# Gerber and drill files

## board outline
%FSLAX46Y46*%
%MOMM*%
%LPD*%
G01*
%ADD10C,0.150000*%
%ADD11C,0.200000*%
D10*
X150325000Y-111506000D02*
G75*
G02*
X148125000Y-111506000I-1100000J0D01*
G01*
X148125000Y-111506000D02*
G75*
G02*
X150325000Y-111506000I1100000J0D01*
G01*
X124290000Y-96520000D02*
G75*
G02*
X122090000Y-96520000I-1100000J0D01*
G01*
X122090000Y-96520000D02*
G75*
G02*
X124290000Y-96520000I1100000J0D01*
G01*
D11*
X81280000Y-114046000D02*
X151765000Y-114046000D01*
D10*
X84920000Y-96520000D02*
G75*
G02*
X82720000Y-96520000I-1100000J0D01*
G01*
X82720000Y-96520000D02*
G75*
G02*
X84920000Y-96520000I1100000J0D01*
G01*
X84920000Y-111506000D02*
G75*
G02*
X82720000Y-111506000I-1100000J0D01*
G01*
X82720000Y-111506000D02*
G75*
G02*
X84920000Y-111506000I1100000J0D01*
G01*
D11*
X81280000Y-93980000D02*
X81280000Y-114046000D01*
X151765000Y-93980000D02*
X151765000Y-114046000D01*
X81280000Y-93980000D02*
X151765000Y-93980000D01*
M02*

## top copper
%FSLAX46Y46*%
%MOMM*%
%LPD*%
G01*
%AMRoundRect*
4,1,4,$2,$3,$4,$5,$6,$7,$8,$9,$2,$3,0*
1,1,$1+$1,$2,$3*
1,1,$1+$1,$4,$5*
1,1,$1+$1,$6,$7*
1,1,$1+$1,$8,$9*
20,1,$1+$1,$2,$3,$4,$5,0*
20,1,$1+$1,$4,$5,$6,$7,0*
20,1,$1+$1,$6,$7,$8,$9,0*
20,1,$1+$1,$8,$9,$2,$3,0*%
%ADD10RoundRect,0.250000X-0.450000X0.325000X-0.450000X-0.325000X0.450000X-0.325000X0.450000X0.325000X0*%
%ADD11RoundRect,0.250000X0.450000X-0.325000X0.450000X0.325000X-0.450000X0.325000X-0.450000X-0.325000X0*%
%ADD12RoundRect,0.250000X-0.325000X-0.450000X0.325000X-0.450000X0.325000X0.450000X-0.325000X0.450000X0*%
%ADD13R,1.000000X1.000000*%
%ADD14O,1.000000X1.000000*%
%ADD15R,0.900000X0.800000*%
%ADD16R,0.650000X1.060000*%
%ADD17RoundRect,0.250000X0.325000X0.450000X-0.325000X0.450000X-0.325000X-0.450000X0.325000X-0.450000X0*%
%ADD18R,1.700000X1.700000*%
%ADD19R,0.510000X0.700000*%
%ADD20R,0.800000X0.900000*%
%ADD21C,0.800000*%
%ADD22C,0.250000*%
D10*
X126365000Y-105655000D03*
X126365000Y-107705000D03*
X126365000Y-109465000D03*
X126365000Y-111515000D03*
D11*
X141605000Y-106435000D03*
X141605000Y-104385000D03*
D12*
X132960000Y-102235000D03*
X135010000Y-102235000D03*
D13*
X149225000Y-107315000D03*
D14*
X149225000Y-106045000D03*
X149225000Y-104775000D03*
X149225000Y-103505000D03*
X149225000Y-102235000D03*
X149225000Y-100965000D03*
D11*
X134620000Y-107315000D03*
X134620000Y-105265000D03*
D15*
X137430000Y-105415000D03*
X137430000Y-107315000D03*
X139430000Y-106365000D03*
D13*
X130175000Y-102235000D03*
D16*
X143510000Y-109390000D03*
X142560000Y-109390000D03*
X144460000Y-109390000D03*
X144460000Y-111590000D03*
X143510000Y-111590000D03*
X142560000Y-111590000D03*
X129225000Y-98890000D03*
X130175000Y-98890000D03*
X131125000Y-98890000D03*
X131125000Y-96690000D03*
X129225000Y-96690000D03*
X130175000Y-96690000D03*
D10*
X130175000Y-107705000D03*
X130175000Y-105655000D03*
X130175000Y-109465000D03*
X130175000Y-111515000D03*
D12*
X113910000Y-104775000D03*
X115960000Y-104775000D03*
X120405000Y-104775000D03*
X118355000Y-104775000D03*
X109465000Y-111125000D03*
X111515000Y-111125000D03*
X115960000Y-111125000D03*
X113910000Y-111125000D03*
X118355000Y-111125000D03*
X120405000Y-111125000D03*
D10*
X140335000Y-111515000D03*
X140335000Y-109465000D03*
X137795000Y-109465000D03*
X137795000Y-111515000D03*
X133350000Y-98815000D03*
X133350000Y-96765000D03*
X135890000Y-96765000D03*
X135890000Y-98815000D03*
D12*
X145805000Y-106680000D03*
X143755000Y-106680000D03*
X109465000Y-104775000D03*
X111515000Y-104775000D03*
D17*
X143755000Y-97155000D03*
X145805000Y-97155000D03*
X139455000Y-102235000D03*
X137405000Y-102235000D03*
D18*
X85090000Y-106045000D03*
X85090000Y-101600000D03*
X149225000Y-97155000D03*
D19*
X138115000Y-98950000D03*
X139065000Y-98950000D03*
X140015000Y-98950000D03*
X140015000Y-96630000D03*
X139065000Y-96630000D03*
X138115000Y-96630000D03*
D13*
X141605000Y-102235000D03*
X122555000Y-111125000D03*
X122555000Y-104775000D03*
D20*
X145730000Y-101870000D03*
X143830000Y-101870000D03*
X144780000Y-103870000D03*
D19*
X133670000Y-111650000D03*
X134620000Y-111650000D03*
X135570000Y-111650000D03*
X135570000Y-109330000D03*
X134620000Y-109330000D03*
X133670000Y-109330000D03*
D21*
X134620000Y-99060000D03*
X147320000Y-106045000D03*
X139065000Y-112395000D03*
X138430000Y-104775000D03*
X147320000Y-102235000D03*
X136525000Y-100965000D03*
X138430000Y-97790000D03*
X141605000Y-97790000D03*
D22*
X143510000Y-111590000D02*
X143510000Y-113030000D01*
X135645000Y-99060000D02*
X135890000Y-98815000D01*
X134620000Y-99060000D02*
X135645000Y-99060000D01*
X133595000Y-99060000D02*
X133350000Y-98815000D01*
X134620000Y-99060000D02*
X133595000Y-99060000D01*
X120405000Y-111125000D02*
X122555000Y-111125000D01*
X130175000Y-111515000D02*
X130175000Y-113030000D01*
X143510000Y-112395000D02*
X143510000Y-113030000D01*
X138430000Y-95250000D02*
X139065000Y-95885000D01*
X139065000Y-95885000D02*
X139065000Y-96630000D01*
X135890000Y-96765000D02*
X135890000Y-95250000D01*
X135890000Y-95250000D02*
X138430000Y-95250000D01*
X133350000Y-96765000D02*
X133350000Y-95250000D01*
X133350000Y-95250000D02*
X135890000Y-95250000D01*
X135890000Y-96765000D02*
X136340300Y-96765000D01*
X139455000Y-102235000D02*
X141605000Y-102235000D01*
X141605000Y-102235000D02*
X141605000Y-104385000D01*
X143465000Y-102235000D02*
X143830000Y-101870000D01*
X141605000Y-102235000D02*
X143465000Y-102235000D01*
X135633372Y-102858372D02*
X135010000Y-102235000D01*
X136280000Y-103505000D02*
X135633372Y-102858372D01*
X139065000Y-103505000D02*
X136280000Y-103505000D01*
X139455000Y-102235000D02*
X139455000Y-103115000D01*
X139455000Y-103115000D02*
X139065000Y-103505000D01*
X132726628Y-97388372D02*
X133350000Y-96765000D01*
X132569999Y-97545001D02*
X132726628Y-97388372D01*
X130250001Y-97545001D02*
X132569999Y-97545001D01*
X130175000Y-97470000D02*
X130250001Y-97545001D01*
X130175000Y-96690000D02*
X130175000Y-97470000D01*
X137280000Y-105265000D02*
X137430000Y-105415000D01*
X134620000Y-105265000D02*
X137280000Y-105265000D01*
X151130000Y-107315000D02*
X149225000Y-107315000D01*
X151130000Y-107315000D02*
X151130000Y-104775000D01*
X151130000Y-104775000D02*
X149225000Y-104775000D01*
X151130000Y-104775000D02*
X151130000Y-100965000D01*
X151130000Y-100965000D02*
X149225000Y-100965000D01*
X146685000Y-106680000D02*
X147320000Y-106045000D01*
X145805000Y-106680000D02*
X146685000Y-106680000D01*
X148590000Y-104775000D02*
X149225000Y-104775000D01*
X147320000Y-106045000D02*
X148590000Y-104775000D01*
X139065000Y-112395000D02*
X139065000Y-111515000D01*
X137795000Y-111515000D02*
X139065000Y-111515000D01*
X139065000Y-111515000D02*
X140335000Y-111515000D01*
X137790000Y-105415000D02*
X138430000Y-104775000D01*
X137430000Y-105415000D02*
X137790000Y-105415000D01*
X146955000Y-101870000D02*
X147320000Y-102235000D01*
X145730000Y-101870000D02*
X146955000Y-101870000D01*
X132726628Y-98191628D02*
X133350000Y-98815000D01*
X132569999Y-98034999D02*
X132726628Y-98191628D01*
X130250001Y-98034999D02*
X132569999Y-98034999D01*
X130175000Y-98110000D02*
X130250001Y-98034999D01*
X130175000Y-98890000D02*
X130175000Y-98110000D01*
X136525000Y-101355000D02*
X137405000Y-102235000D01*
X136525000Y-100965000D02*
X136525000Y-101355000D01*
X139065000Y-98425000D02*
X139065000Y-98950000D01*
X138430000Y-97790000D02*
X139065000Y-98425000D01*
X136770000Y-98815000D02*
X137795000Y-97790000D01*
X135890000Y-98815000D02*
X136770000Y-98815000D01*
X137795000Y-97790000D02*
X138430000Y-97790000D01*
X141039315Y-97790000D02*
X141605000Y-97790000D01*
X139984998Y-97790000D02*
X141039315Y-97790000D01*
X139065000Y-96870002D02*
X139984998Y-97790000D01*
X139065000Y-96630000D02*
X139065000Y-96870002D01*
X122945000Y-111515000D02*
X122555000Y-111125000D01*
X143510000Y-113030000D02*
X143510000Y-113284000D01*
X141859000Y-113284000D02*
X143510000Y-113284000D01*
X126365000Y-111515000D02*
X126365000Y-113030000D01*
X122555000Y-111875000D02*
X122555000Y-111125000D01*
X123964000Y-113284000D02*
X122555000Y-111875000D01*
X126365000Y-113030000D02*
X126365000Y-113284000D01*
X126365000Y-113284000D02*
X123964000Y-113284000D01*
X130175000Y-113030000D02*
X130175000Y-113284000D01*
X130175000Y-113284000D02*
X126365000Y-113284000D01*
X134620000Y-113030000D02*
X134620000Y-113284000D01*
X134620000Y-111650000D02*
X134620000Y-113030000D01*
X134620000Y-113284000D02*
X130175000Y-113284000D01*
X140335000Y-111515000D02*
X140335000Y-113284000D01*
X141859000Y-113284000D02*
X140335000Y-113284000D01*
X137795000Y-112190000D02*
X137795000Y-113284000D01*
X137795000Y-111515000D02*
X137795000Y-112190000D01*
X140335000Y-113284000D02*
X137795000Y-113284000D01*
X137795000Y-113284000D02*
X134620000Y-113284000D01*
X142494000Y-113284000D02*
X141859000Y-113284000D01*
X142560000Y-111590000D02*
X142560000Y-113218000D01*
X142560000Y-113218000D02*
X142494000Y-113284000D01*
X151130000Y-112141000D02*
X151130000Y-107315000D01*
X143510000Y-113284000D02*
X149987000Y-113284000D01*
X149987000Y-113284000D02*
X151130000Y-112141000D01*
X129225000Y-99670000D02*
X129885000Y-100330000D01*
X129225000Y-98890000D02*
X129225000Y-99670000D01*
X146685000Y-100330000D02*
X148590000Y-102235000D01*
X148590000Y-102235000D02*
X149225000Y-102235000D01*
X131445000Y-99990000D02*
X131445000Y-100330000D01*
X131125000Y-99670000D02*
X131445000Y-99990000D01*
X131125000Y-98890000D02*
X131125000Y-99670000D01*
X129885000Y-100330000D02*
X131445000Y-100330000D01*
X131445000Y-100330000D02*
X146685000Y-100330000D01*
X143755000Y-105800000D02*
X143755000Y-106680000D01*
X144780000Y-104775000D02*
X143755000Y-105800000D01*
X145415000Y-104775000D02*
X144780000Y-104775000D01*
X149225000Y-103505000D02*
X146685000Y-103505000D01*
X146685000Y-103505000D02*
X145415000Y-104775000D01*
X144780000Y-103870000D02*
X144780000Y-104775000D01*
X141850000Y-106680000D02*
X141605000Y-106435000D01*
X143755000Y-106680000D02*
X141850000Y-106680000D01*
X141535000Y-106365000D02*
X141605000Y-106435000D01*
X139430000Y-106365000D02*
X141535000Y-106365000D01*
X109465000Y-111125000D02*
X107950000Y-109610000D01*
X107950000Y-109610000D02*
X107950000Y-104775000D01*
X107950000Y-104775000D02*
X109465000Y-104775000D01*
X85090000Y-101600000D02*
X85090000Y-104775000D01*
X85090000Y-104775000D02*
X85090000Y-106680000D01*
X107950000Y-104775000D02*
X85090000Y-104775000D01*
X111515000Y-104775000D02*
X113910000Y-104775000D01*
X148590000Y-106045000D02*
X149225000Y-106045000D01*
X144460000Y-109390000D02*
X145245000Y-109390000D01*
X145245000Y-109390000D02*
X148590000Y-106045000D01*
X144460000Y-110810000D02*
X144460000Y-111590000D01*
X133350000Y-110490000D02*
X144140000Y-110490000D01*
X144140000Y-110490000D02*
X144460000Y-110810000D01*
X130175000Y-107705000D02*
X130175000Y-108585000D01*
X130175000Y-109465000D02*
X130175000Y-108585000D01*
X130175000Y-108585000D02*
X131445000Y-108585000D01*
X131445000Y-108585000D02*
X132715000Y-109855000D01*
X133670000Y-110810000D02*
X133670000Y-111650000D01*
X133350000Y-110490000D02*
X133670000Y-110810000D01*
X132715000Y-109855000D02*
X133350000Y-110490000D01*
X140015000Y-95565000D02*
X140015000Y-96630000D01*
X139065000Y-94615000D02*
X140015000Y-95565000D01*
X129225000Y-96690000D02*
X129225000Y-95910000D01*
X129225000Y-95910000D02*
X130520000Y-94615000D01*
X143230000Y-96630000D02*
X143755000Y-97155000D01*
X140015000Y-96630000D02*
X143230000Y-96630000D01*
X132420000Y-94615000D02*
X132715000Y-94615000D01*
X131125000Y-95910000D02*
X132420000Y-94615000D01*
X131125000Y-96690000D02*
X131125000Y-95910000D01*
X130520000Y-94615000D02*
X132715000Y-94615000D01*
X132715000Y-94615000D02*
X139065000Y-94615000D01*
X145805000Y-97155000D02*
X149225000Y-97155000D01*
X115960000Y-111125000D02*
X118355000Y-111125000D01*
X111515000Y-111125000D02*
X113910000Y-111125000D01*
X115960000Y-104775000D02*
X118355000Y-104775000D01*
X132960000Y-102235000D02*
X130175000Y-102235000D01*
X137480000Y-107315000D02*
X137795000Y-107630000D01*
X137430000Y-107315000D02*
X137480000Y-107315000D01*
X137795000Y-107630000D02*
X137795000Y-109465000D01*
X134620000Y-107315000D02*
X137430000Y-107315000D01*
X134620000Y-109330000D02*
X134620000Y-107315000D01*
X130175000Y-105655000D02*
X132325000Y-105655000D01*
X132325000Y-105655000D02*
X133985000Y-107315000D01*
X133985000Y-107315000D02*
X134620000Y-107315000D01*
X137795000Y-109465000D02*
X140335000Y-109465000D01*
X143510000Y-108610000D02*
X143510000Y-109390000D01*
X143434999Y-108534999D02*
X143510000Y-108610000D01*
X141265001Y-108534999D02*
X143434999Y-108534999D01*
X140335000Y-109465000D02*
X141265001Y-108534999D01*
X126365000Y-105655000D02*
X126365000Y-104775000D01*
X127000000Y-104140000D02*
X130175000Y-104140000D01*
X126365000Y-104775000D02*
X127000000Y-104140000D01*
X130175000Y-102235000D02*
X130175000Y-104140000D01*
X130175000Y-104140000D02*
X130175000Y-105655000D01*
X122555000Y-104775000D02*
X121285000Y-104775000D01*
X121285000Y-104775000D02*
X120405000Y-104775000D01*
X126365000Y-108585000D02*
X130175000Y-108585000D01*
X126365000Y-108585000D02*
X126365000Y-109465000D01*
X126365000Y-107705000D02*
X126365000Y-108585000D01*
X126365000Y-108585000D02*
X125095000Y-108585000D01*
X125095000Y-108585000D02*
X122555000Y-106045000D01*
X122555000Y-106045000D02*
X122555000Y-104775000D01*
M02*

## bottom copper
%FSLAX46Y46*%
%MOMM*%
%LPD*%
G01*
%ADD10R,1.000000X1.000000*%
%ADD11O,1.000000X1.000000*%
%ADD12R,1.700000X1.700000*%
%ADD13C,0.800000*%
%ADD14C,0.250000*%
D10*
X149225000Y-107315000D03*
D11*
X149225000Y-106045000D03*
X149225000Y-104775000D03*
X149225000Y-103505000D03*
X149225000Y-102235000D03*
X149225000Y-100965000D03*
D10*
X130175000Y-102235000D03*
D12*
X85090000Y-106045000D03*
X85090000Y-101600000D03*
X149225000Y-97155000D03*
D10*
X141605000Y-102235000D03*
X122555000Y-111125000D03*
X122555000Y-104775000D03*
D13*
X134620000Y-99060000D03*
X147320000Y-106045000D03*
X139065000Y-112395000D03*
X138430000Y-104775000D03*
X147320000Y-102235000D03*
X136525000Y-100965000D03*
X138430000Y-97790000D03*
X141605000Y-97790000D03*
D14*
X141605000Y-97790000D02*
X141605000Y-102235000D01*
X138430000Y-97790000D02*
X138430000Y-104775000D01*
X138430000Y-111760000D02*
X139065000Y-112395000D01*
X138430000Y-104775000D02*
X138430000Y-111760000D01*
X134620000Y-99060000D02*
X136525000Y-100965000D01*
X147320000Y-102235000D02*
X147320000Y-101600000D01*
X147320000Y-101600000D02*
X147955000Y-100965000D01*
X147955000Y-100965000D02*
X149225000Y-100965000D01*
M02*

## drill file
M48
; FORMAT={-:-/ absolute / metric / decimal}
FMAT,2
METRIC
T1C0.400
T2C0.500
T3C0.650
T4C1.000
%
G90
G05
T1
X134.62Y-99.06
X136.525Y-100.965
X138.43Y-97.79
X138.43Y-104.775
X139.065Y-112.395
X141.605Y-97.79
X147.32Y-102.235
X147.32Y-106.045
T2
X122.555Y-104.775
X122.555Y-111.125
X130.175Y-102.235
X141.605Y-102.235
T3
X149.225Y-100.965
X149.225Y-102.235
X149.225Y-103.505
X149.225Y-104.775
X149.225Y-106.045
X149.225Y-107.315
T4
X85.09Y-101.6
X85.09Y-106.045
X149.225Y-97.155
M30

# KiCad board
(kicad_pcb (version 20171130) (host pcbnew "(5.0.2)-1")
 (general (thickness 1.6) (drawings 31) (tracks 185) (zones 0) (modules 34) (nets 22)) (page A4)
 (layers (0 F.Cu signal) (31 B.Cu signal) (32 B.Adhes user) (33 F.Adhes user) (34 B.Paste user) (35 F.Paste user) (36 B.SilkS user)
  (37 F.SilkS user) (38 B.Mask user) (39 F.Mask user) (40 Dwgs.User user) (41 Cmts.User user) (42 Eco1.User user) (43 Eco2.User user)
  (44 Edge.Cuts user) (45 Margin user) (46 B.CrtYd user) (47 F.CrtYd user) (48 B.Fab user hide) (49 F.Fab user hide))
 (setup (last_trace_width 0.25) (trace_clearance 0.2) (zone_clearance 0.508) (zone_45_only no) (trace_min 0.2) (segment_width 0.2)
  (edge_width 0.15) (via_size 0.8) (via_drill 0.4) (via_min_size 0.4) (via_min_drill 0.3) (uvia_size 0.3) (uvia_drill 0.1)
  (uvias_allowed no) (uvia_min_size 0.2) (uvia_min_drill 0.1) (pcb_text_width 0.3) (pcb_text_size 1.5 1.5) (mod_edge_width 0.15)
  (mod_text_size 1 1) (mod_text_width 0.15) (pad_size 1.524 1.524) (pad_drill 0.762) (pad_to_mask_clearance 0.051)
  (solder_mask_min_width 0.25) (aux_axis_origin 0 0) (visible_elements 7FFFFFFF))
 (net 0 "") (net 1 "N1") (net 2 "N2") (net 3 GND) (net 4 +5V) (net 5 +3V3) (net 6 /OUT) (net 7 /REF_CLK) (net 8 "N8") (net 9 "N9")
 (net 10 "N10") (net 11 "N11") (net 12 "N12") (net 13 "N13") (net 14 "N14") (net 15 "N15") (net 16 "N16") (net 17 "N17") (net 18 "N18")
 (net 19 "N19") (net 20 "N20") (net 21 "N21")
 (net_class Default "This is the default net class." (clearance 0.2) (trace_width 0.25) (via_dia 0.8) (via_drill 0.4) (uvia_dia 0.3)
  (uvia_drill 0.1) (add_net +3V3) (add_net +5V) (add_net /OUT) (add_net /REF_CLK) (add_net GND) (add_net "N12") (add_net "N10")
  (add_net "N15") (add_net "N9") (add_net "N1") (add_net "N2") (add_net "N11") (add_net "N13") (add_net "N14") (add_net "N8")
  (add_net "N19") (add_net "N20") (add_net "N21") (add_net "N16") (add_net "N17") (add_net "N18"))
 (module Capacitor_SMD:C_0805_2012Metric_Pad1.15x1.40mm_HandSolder (layer F.Cu) (at 126.365 106.68 270)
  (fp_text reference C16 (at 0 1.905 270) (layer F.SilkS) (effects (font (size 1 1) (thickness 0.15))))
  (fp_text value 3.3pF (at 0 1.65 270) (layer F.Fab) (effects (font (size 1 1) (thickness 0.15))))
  (pad 1 smd roundrect (at -1.025 0 270) (size 1.15 1.4) (layers F.Cu F.Paste F.Mask) (roundrect_rratio 0.217391) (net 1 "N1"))
  (pad 2 smd roundrect (at 1.025 0 270) (size 1.15 1.4) (layers F.Cu F.Paste F.Mask) (roundrect_rratio 0.217391) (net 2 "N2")))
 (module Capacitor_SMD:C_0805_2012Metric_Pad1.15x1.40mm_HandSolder (layer F.Cu) (at 126.365 110.49 270)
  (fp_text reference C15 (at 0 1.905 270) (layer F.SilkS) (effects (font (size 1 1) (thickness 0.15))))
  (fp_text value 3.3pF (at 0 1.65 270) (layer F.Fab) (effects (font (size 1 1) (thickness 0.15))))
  (pad 1 smd roundrect (at -1.025 0 270) (size 1.15 1.4) (layers F.Cu F.Paste F.Mask) (roundrect_rratio 0.217391) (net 2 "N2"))
  (pad 2 smd roundrect (at 1.025 0 270) (size 1.15 1.4) (layers F.Cu F.Paste F.Mask) (roundrect_rratio 0.217391) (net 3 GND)))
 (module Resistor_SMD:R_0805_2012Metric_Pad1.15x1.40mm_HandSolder (layer F.Cu) (at 141.605 105.41 90)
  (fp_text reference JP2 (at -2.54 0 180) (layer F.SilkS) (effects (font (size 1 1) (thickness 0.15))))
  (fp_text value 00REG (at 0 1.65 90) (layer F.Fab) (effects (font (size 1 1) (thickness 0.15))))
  (pad 1 smd roundrect (at -1.025 0 90) (size 1.15 1.4) (layers F.Cu F.Paste F.Mask) (roundrect_rratio 0.217391) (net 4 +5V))
  (pad 2 smd roundrect (at 1.025 0 90) (size 1.15 1.4) (layers F.Cu F.Paste F.Mask) (roundrect_rratio 0.217391) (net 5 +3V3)))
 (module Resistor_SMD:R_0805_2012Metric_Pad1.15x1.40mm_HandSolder (layer F.Cu) (at 133.985 102.235)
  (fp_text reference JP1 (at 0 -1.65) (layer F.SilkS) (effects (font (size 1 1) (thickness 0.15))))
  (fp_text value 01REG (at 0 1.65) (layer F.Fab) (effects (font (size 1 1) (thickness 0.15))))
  (pad 1 smd roundrect (at -1.025 0) (size 1.15 1.4) (layers F.Cu F.Paste F.Mask) (roundrect_rratio 0.217391) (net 1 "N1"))
  (pad 2 smd roundrect (at 1.025 0) (size 1.15 1.4) (layers F.Cu F.Paste F.Mask) (roundrect_rratio 0.217391) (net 5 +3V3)))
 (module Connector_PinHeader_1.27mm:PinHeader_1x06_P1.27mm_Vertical (layer F.Cu) (at 149.225 107.315 180)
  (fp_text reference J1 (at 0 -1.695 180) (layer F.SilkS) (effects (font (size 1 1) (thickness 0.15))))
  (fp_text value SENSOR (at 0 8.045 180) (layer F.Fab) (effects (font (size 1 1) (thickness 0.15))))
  (pad 1 thru_hole rect (at 0 0 180) (size 1 1) (drill 0.65) (layers *.Cu *.Mask) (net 3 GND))
  (pad 2 thru_hole oval (at 0 1.27 180) (size 1 1) (drill 0.65) (layers *.Cu *.Mask) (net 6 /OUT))
  (pad 3 thru_hole oval (at 0 2.54 180) (size 1 1) (drill 0.65) (layers *.Cu *.Mask) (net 3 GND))
  (pad 4 thru_hole oval (at 0 3.81 180) (size 1 1) (drill 0.65) (layers *.Cu *.Mask) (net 4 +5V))
  (pad 5 thru_hole oval (at 0 5.08 180) (size 1 1) (drill 0.65) (layers *.Cu *.Mask) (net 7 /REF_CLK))
  (pad 6 thru_hole oval (at 0 6.35 180) (size 1 1) (drill 0.65) (layers *.Cu *.Mask) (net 3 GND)))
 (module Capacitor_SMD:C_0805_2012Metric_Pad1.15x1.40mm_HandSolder (layer F.Cu) (at 134.62 106.29 90)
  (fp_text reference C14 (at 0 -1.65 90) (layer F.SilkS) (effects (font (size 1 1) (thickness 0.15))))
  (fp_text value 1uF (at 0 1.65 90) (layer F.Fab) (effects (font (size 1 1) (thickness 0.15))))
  (pad 1 smd roundrect (at -1.025 0 90) (size 1.15 1.4) (layers F.Cu F.Paste F.Mask) (roundrect_rratio 0.217391) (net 1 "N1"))
  (pad 2 smd roundrect (at 1.025 0 90) (size 1.15 1.4) (layers F.Cu F.Paste F.Mask) (roundrect_rratio 0.217391) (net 3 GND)))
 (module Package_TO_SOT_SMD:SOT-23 (layer F.Cu) (at 138.43 106.365)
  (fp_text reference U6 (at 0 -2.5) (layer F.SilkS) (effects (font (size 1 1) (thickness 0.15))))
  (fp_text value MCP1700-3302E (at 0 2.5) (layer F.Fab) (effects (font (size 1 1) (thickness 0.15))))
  (pad 1 smd rect (at -1 -0.95) (size 0.9 0.8) (layers F.Cu F.Paste F.Mask) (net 3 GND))
  (pad 2 smd rect (at -1 0.95) (size 0.9 0.8) (layers F.Cu F.Paste F.Mask) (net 1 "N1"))
  (pad 3 smd rect (at 1 0) (size 0.9 0.8) (layers F.Cu F.Paste F.Mask) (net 4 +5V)))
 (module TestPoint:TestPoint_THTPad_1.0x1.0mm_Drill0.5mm (layer F.Cu) (at 130.175 102.235)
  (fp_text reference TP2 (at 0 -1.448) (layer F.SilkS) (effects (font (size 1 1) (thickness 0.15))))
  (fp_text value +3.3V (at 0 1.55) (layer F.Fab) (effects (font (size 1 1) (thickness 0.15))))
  (pad 1 thru_hole rect (at 0 0) (size 1 1) (drill 0.5) (layers *.Cu *.Mask) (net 1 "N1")))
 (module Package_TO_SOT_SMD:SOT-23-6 (layer F.Cu) (at 143.51 110.49 90)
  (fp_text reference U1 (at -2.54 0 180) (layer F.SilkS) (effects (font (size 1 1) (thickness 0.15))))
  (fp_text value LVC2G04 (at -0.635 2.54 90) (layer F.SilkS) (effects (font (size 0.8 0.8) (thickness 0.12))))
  (pad 5 smd rect (at 1.1 0 90) (size 1.06 0.65) (layers F.Cu F.Paste F.Mask) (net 1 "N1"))
  (pad 6 smd rect (at 1.1 -0.95 90) (size 1.06 0.65) (layers F.Cu F.Paste F.Mask) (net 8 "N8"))
  (pad 4 smd rect (at 1.1 0.95 90) (size 1.06 0.65) (layers F.Cu F.Paste F.Mask) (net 6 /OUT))
  (pad 3 smd rect (at -1.1 0.95 90) (size 1.06 0.65) (layers F.Cu F.Paste F.Mask) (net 2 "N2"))
  (pad 2 smd rect (at -1.1 0 90) (size 1.06 0.65) (layers F.Cu F.Paste F.Mask) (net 3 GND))
  (pad 1 smd rect (at -1.1 -0.95 90) (size 1.06 0.65) (layers F.Cu F.Paste F.Mask) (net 3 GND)))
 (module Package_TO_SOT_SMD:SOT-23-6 (layer F.Cu) (at 130.175 97.79 90)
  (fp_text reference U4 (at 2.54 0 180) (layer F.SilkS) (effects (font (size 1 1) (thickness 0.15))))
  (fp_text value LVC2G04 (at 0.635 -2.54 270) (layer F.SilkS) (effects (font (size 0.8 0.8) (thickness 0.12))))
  (pad 1 smd rect (at -1.1 -0.95 90) (size 1.06 0.65) (layers F.Cu F.Paste F.Mask) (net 7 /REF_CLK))
  (pad 2 smd rect (at -1.1 0 90) (size 1.06 0.65) (layers F.Cu F.Paste F.Mask) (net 3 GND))
  (pad 3 smd rect (at -1.1 0.95 90) (size 1.06 0.65) (layers F.Cu F.Paste F.Mask) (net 7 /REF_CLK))
  (pad 4 smd rect (at 1.1 0.95 90) (size 1.06 0.65) (layers F.Cu F.Paste F.Mask) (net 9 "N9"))
  (pad 6 smd rect (at 1.1 -0.95 90) (size 1.06 0.65) (layers F.Cu F.Paste F.Mask) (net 9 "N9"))
  (pad 5 smd rect (at 1.1 0 90) (size 1.06 0.65) (layers F.Cu F.Paste F.Mask) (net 5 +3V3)))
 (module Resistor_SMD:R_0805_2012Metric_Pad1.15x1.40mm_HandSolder (layer F.Cu) (at 130.175 106.68 270)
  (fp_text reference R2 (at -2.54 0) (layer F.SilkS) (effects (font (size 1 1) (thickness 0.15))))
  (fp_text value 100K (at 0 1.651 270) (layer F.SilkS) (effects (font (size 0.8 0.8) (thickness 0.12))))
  (pad 2 smd roundrect (at 1.025 0 270) (size 1.15 1.4) (layers F.Cu F.Paste F.Mask) (roundrect_rratio 0.217391) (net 2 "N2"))
  (pad 1 smd roundrect (at -1.025 0 270) (size 1.15 1.4) (layers F.Cu F.Paste F.Mask) (roundrect_rratio 0.217391) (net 1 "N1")))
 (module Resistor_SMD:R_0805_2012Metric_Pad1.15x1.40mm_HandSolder (layer F.Cu) (at 130.175 110.49 270)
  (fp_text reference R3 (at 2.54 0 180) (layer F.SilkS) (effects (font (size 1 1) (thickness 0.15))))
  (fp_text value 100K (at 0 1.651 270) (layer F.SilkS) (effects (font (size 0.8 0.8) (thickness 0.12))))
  (pad 1 smd roundrect (at -1.025 0 270) (size 1.15 1.4) (layers F.Cu F.Paste F.Mask) (roundrect_rratio 0.217391) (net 2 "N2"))
  (pad 2 smd roundrect (at 1.025 0 270) (size 1.15 1.4) (layers F.Cu F.Paste F.Mask) (roundrect_rratio 0.217391) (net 3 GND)))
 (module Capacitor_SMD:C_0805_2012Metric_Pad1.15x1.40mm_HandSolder (layer F.Cu) (at 114.935 104.775)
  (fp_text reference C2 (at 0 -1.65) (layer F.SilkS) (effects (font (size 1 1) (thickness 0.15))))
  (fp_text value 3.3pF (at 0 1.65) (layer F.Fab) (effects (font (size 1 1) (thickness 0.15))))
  (pad 1 smd roundrect (at -1.025 0) (size 1.15 1.4) (layers F.Cu F.Paste F.Mask) (roundrect_rratio 0.217391) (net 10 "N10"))
  (pad 2 smd roundrect (at 1.025 0) (size 1.15 1.4) (layers F.Cu F.Paste F.Mask) (roundrect_rratio 0.217391) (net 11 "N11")))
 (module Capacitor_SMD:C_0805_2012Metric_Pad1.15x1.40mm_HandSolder (layer F.Cu) (at 119.38 104.775)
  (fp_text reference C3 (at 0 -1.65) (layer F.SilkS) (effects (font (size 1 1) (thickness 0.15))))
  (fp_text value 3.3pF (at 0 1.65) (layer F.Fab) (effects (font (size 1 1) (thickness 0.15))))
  (pad 2 smd roundrect (at 1.025 0) (size 1.15 1.4) (layers F.Cu F.Paste F.Mask) (roundrect_rratio 0.217391) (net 2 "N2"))
  (pad 1 smd roundrect (at -1.025 0) (size 1.15 1.4) (layers F.Cu F.Paste F.Mask) (roundrect_rratio 0.217391) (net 11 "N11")))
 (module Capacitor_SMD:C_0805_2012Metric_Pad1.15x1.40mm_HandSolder (layer F.Cu) (at 110.49 111.125)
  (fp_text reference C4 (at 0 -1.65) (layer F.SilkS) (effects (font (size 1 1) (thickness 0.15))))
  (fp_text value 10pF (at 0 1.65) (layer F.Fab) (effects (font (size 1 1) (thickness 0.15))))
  (pad 1 smd roundrect (at -1.025 0) (size 1.15 1.4) (layers F.Cu F.Paste F.Mask) (roundrect_rratio 0.217391) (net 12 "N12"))
  (pad 2 smd roundrect (at 1.025 0) (size 1.15 1.4) (layers F.Cu F.Paste F.Mask) (roundrect_rratio 0.217391) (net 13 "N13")))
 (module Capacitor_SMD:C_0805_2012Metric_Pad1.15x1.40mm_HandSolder (layer F.Cu) (at 114.935 111.125)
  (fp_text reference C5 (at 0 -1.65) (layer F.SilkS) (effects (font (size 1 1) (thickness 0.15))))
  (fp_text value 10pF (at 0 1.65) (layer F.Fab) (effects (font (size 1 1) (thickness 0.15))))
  (pad 2 smd roundrect (at 1.025 0) (size 1.15 1.4) (layers F.Cu F.Paste F.Mask) (roundrect_rratio 0.217391) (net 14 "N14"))
  (pad 1 smd roundrect (at -1.025 0) (size 1.15 1.4) (layers F.Cu F.Paste F.Mask) (roundrect_rratio 0.217391) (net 13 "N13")))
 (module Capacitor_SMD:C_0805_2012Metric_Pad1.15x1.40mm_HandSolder (layer F.Cu) (at 119.38 111.125)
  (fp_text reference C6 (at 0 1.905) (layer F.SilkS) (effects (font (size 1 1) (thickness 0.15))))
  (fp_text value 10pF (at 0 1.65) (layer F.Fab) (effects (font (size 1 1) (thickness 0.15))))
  (pad 1 smd roundrect (at -1.025 0) (size 1.15 1.4) (layers F.Cu F.Paste F.Mask) (roundrect_rratio 0.217391) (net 14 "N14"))
  (pad 2 smd roundrect (at 1.025 0) (size 1.15 1.4) (layers F.Cu F.Paste F.Mask) (roundrect_rratio 0.217391) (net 3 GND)))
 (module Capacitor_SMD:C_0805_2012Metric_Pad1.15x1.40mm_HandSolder (layer F.Cu) (at 140.335 110.49 270)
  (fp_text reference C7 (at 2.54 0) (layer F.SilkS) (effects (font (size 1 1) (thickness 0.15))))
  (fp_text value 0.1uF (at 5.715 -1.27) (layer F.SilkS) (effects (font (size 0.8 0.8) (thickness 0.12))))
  (pad 2 smd roundrect (at 1.025 0 270) (size 1.15 1.4) (layers F.Cu F.Paste F.Mask) (roundrect_rratio 0.217391) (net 3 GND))
  (pad 1 smd roundrect (at -1.025 0 270) (size 1.15 1.4) (layers F.Cu F.Paste F.Mask) (roundrect_rratio 0.217391) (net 1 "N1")))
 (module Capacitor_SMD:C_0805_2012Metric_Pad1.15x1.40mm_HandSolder (layer F.Cu) (at 137.795 110.49 270)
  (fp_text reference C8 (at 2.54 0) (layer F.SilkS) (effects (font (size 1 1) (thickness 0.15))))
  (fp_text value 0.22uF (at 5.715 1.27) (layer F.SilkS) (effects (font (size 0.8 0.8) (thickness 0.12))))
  (pad 1 smd roundrect (at -1.025 0 270) (size 1.15 1.4) (layers F.Cu F.Paste F.Mask) (roundrect_rratio 0.217391) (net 1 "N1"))
  (pad 2 smd roundrect (at 1.025 0 270) (size 1.15 1.4) (layers F.Cu F.Paste F.Mask) (roundrect_rratio 0.217391) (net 3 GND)))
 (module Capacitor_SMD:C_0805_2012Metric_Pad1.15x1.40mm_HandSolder (layer F.Cu) (at 133.35 97.79 270)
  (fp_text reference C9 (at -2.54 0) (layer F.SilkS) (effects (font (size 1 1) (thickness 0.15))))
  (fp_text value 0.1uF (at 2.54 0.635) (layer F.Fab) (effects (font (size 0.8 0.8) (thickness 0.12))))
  (pad 2 smd roundrect (at 1.025 0 270) (size 1.15 1.4) (layers F.Cu F.Paste F.Mask) (roundrect_rratio 0.217391) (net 3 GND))
  (pad 1 smd roundrect (at -1.025 0 270) (size 1.15 1.4) (layers F.Cu F.Paste F.Mask) (roundrect_rratio 0.217391) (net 5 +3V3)))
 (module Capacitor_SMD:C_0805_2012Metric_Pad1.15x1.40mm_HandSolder (layer F.Cu) (at 135.89 97.79 270)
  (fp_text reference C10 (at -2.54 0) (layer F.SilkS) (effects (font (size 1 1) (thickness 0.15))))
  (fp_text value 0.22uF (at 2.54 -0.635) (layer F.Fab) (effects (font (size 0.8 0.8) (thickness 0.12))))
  (pad 1 smd roundrect (at -1.025 0 270) (size 1.15 1.4) (layers F.Cu F.Paste F.Mask) (roundrect_rratio 0.217391) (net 5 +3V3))
  (pad 2 smd roundrect (at 1.025 0 270) (size 1.15 1.4) (layers F.Cu F.Paste F.Mask) (roundrect_rratio 0.217391) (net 3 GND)))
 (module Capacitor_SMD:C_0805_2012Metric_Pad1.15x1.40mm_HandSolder (layer F.Cu) (at 144.78 106.68)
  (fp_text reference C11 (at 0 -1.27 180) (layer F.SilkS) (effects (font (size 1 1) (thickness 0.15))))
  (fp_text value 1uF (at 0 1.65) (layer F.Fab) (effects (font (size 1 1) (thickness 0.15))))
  (pad 2 smd roundrect (at 1.025 0) (size 1.15 1.4) (layers F.Cu F.Paste F.Mask) (roundrect_rratio 0.217391) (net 3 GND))
  (pad 1 smd roundrect (at -1.025 0) (size 1.15 1.4) (layers F.Cu F.Paste F.Mask) (roundrect_rratio 0.217391) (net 4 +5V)))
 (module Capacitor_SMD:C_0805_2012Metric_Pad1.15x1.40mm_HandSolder (layer F.Cu) (at 110.49 104.775)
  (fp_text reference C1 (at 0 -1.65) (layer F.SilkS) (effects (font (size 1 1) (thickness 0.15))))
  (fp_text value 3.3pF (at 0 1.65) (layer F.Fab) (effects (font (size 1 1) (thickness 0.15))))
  (pad 1 smd roundrect (at -1.025 0) (size 1.15 1.4) (layers F.Cu F.Paste F.Mask) (roundrect_rratio 0.217391) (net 12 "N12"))
  (pad 2 smd roundrect (at 1.025 0) (size 1.15 1.4) (layers F.Cu F.Paste F.Mask) (roundrect_rratio 0.217391) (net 10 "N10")))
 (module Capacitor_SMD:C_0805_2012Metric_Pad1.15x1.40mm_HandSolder (layer F.Cu) (at 144.78 97.155 180)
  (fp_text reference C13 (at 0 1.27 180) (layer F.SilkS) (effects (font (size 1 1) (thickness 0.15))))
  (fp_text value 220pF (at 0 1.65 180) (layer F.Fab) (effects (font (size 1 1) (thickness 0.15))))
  (pad 2 smd roundrect (at 1.025 0 180) (size 1.15 1.4) (layers F.Cu F.Paste F.Mask) (roundrect_rratio 0.217391) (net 9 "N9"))
  (pad 1 smd roundrect (at -1.025 0 180) (size 1.15 1.4) (layers F.Cu F.Paste F.Mask) (roundrect_rratio 0.217391) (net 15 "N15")))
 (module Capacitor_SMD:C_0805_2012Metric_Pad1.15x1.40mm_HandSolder (layer F.Cu) (at 138.43 102.235 180)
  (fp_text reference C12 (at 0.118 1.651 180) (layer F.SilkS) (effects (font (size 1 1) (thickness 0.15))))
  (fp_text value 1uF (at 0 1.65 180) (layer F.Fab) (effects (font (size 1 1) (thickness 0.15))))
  (pad 1 smd roundrect (at -1.025 0 180) (size 1.15 1.4) (layers F.Cu F.Paste F.Mask) (roundrect_rratio 0.217391) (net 5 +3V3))
  (pad 2 smd roundrect (at 1.025 0 180) (size 1.15 1.4) (layers F.Cu F.Paste F.Mask) (roundrect_rratio 0.217391) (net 3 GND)))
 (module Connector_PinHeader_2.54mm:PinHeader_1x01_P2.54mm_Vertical (layer F.Cu) (at 85.09 106.045)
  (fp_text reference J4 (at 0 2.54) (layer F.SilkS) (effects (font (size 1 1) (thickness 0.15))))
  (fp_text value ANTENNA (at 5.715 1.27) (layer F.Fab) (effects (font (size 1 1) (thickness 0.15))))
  (pad 1 thru_hole rect (at 0 0) (size 1.7 1.7) (drill 1) (layers *.Cu *.Mask) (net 12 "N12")))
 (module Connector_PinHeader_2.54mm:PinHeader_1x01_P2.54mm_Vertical (layer F.Cu) (at 85.09 101.6 180)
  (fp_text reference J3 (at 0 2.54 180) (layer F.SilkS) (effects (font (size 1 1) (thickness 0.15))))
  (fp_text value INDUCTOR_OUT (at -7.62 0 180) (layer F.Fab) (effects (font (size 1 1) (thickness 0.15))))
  (pad 1 thru_hole rect (at 0 0 180) (size 1.7 1.7) (drill 1) (layers *.Cu *.Mask) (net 12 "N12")))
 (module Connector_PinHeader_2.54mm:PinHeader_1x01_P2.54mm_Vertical (layer F.Cu) (at 149.225 97.155 180)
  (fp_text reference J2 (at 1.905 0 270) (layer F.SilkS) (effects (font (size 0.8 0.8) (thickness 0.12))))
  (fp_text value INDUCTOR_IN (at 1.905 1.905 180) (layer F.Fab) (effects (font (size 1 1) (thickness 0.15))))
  (pad 1 thru_hole rect (at 0 0 180) (size 1.7 1.7) (drill 1) (layers *.Cu *.Mask) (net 15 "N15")))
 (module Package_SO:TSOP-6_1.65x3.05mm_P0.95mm (layer F.Cu) (at 139.065 97.79 90)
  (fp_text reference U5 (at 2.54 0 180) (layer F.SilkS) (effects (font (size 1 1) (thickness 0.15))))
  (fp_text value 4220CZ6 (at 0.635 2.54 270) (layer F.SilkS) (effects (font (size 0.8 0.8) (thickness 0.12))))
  (pad 1 smd rect (at -1.16 -0.95 90) (size 0.7 0.51) (layers F.Cu F.Paste F.Mask) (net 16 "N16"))
  (pad 2 smd rect (at -1.16 0 90) (size 0.7 0.51) (layers F.Cu F.Paste F.Mask) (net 3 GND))
  (pad 3 smd rect (at -1.16 0.95 90) (size 0.7 0.51) (layers F.Cu F.Paste F.Mask) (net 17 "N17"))
  (pad 4 smd rect (at 1.16 0.95 90) (size 0.7 0.51) (layers F.Cu F.Paste F.Mask) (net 9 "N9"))
  (pad 5 smd rect (at 1.16 0 90) (size 0.7 0.51) (layers F.Cu F.Paste F.Mask) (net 5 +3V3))
  (pad 6 smd rect (at 1.16 -0.95 90) (size 0.7 0.51) (layers F.Cu F.Paste F.Mask) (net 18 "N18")))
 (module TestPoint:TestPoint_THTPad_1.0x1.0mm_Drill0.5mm (layer F.Cu) (at 141.605 102.235 180)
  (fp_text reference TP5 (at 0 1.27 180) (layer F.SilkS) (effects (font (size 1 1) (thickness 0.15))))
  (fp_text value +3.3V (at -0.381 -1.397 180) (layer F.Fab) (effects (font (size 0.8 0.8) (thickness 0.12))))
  (pad 1 thru_hole rect (at 0 0 180) (size 1 1) (drill 0.5) (layers *.Cu *.Mask) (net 5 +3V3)))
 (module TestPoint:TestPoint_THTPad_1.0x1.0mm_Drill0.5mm (layer F.Cu) (at 122.555 111.125)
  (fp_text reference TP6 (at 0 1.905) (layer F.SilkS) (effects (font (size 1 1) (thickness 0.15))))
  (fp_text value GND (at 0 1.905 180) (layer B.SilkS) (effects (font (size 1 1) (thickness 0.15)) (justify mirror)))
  (pad 1 thru_hole rect (at 0 0) (size 1 1) (drill 0.5) (layers *.Cu *.Mask) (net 3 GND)))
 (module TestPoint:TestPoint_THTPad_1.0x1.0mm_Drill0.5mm (layer F.Cu) (at 122.555 104.775)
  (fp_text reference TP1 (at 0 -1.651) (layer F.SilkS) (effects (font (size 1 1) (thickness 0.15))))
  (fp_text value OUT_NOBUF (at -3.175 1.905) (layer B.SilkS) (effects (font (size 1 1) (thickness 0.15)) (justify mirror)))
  (pad 1 thru_hole rect (at 0 0) (size 1 1) (drill 0.5) (layers *.Cu *.Mask) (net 2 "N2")))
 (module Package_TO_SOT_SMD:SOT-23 (layer F.Cu) (at 144.78 102.87 270)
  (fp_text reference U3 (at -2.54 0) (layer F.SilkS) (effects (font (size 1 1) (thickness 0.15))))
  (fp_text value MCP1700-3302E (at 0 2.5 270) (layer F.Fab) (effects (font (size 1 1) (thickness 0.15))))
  (pad 1 smd rect (at -1 -0.95 270) (size 0.9 0.8) (layers F.Cu F.Paste F.Mask) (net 3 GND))
  (pad 2 smd rect (at -1 0.95 270) (size 0.9 0.8) (layers F.Cu F.Paste F.Mask) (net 5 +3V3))
  (pad 3 smd rect (at 1 0 270) (size 0.9 0.8) (layers F.Cu F.Paste F.Mask) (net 4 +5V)))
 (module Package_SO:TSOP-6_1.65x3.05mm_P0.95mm (layer F.Cu) (at 134.62 110.49 90)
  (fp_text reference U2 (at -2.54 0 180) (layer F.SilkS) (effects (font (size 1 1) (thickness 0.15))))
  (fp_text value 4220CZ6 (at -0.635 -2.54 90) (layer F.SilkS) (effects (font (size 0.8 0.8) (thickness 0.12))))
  (pad 1 smd rect (at -1.16 -0.95 90) (size 0.7 0.51) (layers F.Cu F.Paste F.Mask) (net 2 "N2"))
  (pad 2 smd rect (at -1.16 0 90) (size 0.7 0.51) (layers F.Cu F.Paste F.Mask) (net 3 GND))
  (pad 3 smd rect (at -1.16 0.95 90) (size 0.7 0.51) (layers F.Cu F.Paste F.Mask) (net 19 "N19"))
  (pad 4 smd rect (at 1.16 0.95 90) (size 0.7 0.51) (layers F.Cu F.Paste F.Mask) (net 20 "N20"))
  (pad 5 smd rect (at 1.16 0 90) (size 0.7 0.51) (layers F.Cu F.Paste F.Mask) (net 1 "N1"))
  (pad 6 smd rect (at 1.16 -0.95 90) (size 0.7 0.51) (layers F.Cu F.Paste F.Mask) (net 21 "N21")))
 (gr_circle (center 149.225 111.506) (end 150.325 111.506) (layer Edge.Cuts) (width 0.15))
 (gr_circle (center 123.19 96.52) (end 124.29 96.52) (layer Edge.Cuts) (width 0.15))
 (gr_line (start 81.28 114.046) (end 151.765 114.046) (layer Edge.Cuts) (width 0.2))
 (gr_circle (center 83.82 96.52) (end 84.92 96.52) (layer Edge.Cuts) (width 0.15))
 (gr_circle (center 83.82 111.506) (end 84.92 111.506) (layer Edge.Cuts) (width 0.15))
 (gr_line (start 81.28 93.98) (end 81.28 114.046) (layer Edge.Cuts) (width 0.2))
 (gr_line (start 151.765 93.98) (end 151.765 114.046) (layer Edge.Cuts) (width 0.2))
 (gr_line (start 81.28 93.98) (end 151.765 93.98) (layer Edge.Cuts) (width 0.2))
 (segment (start 143.51 111.59) (end 143.51 113.03) (width 0.25) (layer F.Cu) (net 3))
 (via (at 134.62 99.06) (size 0.8) (drill 0.4) (layers F.Cu B.Cu) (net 3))
 (segment (start 135.645 99.06) (end 135.89 98.815) (width 0.25) (layer F.Cu) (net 3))
 (segment (start 134.62 99.06) (end 135.645 99.06) (width 0.25) (layer F.Cu) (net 3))
 (segment (start 133.595 99.06) (end 133.35 98.815) (width 0.25) (layer F.Cu) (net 3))
 (segment (start 134.62 99.06) (end 133.595 99.06) (width 0.25) (layer F.Cu) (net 3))
 (segment (start 120.405 111.125) (end 122.555 111.125) (width 0.25) (layer F.Cu) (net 3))
 (segment (start 130.175 111.515) (end 130.175 113.03) (width 0.25) (layer F.Cu) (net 3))
 (segment (start 143.51 112.395) (end 143.51 113.03) (width 0.25) (layer F.Cu) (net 3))
 (segment (start 138.43 95.25) (end 139.065 95.885) (width 0.25) (layer F.Cu) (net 5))
 (segment (start 139.065 95.885) (end 139.065 96.63) (width 0.25) (layer F.Cu) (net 5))
 (segment (start 135.89 96.765) (end 135.89 95.25) (width 0.25) (layer F.Cu) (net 5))
 (segment (start 135.89 95.25) (end 138.43 95.25) (width 0.25) (layer F.Cu) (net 5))
 (segment (start 133.35 96.765) (end 133.35 95.25) (width 0.25) (layer F.Cu) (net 5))
 (segment (start 133.35 95.25) (end 135.89 95.25) (width 0.25) (layer F.Cu) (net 5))
 (segment (start 135.89 96.765) (end 136.3403 96.765) (width 0.25) (layer F.Cu) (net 5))
 (segment (start 139.455 102.235) (end 141.605 102.235) (width 0.25) (layer F.Cu) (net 5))
 (segment (start 141.605 102.235) (end 141.605 104.385) (width 0.25) (layer F.Cu) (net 5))
 (segment (start 143.465 102.235) (end 143.83 101.87) (width 0.25) (layer F.Cu) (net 5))
 (segment (start 141.605 102.235) (end 143.465 102.235) (width 0.25) (layer F.Cu) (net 5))
 (segment (start 135.633372 102.858372) (end 135.01 102.235) (width 0.25) (layer F.Cu) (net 5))
 (segment (start 136.28 103.505) (end 135.633372 102.858372) (width 0.25) (layer F.Cu) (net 5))
 (segment (start 139.065 103.505) (end 136.28 103.505) (width 0.25) (layer F.Cu) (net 5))
 (segment (start 139.455 102.235) (end 139.455 103.115) (width 0.25) (layer F.Cu) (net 5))
 (segment (start 139.455 103.115) (end 139.065 103.505) (width 0.25) (layer F.Cu) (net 5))
 (segment (start 132.726628 97.388372) (end 133.35 96.765) (width 0.25) (layer F.Cu) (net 5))
 (segment (start 132.569999 97.545001) (end 132.726628 97.388372) (width 0.25) (layer F.Cu) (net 5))
 (segment (start 130.250001 97.545001) (end 132.569999 97.545001) (width 0.25) (layer F.Cu) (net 5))
 (segment (start 130.175 97.47) (end 130.250001 97.545001) (width 0.25) (layer F.Cu) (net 5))
 (segment (start 130.175 96.69) (end 130.175 97.47) (width 0.25) (layer F.Cu) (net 5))
 (segment (start 137.28 105.265) (end 137.43 105.415) (width 0.25) (layer F.Cu) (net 3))
 (segment (start 134.62 105.265) (end 137.28 105.265) (width 0.25) (layer F.Cu) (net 3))
 (segment (start 151.13 107.315) (end 149.225 107.315) (width 0.25) (layer F.Cu) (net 3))
 (segment (start 151.13 107.315) (end 151.13 104.775) (width 0.25) (layer F.Cu) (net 3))
 (segment (start 151.13 104.775) (end 149.225 104.775) (width 0.25) (layer F.Cu) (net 3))
 (segment (start 151.13 104.775) (end 151.13 100.965) (width 0.25) (layer F.Cu) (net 3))
 (segment (start 151.13 100.965) (end 149.225 100.965) (width 0.25) (layer F.Cu) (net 3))
 (via (at 147.32 106.045) (size 0.8) (drill 0.4) (layers F.Cu B.Cu) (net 3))
 (segment (start 146.685 106.68) (end 147.32 106.045) (width 0.25) (layer F.Cu) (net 3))
 (segment (start 145.805 106.68) (end 146.685 106.68) (width 0.25) (layer F.Cu) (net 3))
 (via (at 139.065 112.395) (size 0.8) (drill 0.4) (layers F.Cu B.Cu) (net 3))
 (segment (start 148.59 104.775) (end 149.225 104.775) (width 0.25) (layer F.Cu) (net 3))
 (segment (start 147.32 106.045) (end 148.59 104.775) (width 0.25) (layer F.Cu) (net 3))
 (segment (start 139.065 112.395) (end 139.065 111.515) (width 0.25) (layer F.Cu) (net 3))
 (segment (start 137.795 111.515) (end 139.065 111.515) (width 0.25) (layer F.Cu) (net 3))
 (segment (start 139.065 111.515) (end 140.335 111.515) (width 0.25) (layer F.Cu) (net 3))
 (via (at 138.43 104.775) (size 0.8) (drill 0.4) (layers F.Cu B.Cu) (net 3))
 (segment (start 137.79 105.415) (end 138.43 104.775) (width 0.25) (layer F.Cu) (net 3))
 (segment (start 137.43 105.415) (end 137.79 105.415) (width 0.25) (layer F.Cu) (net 3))
 (via (at 147.32 102.235) (size 0.8) (drill 0.4) (layers F.Cu B.Cu) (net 3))
 (segment (start 146.955 101.87) (end 147.32 102.235) (width 0.25) (layer F.Cu) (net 3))
 (segment (start 145.73 101.87) (end 146.955 101.87) (width 0.25) (layer F.Cu) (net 3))
 (segment (start 132.726628 98.191628) (end 133.35 98.815) (width 0.25) (layer F.Cu) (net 3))
 (segment (start 132.569999 98.034999) (end 132.726628 98.191628) (width 0.25) (layer F.Cu) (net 3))
 (segment (start 130.250001 98.034999) (end 132.569999 98.034999) (width 0.25) (layer F.Cu) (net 3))
 (segment (start 130.175 98.11) (end 130.250001 98.034999) (width 0.25) (layer F.Cu) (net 3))
 (segment (start 130.175 98.89) (end 130.175 98.11) (width 0.25) (layer F.Cu) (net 3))
 (via (at 136.525 100.965) (size 0.8) (drill 0.4) (layers F.Cu B.Cu) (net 3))
 (segment (start 136.525 101.355) (end 137.405 102.235) (width 0.25) (layer F.Cu) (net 3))
 (segment (start 136.525 100.965) (end 136.525 101.355) (width 0.25) (layer F.Cu) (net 3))
 (via (at 138.43 97.79) (size 0.8) (drill 0.4) (layers F.Cu B.Cu) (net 3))
 (segment (start 139.065 98.425) (end 139.065 98.95) (width 0.25) (layer F.Cu) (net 3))
 (segment (start 138.43 97.79) (end 139.065 98.425) (width 0.25) (layer F.Cu) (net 3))
 (segment (start 136.77 98.815) (end 137.795 97.79) (width 0.25) (layer F.Cu) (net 3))
 (segment (start 135.89 98.815) (end 136.77 98.815) (width 0.25) (layer F.Cu) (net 3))
 (segment (start 137.795 97.79) (end 138.43 97.79) (width 0.25) (layer F.Cu) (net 3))
 (via (at 141.605 97.79) (size 0.8) (drill 0.4) (layers F.Cu B.Cu) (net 5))
 (segment (start 141.039315 97.79) (end 141.605 97.79) (width 0.25) (layer F.Cu) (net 5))
 (segment (start 139.984998 97.79) (end 141.039315 97.79) (width 0.25) (layer F.Cu) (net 5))
 (segment (start 139.065 96.870002) (end 139.984998 97.79) (width 0.25) (layer F.Cu) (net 5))
 (segment (start 139.065 96.63) (end 139.065 96.870002) (width 0.25) (layer F.Cu) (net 5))
 (segment (start 141.605 97.79) (end 141.605 102.235) (width 0.25) (layer B.Cu) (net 5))
 (segment (start 138.43 97.79) (end 138.43 104.775) (width 0.25) (layer B.Cu) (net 3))
 (segment (start 138.43 111.76) (end 139.065 112.395) (width 0.25) (layer B.Cu) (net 3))
 (segment (start 138.43 104.775) (end 138.43 111.76) (width 0.25) (layer B.Cu) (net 3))
 (segment (start 134.62 99.06) (end 136.525 100.965) (width 0.25) (layer B.Cu) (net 3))
 (segment (start 147.32 102.235) (end 147.32 101.6) (width 0.25) (layer B.Cu) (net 3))
 (segment (start 147.32 101.6) (end 147.955 100.965) (width 0.25) (layer B.Cu) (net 3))
 (segment (start 147.955 100.965) (end 149.225 100.965) (width 0.25) (layer B.Cu) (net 3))
 (segment (start 122.945 111.515) (end 122.555 111.125) (width 0.25) (layer F.Cu) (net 3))
 (segment (start 143.51 113.03) (end 143.51 113.284) (width 0.25) (layer F.Cu) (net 3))
 (segment (start 141.859 113.284) (end 143.51 113.284) (width 0.25) (layer F.Cu) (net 3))
 (segment (start 126.365 111.515) (end 126.365 113.03) (width 0.25) (layer F.Cu) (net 3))
 (segment (start 122.555 111.875) (end 122.555 111.125) (width 0.25) (layer F.Cu) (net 3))
 (segment (start 123.964 113.284) (end 122.555 111.875) (width 0.25) (layer F.Cu) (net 3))
 (segment (start 126.365 113.03) (end 126.365 113.284) (width 0.25) (layer F.Cu) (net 3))
 (segment (start 126.365 113.284) (end 123.964 113.284) (width 0.25) (layer F.Cu) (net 3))
 (segment (start 130.175 113.03) (end 130.175 113.284) (width 0.25) (layer F.Cu) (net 3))
 (segment (start 130.175 113.284) (end 126.365 113.284) (width 0.25) (layer F.Cu) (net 3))
 (segment (start 134.62 113.03) (end 134.62 113.284) (width 0.25) (layer F.Cu) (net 3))
 (segment (start 134.62 111.65) (end 134.62 113.03) (width 0.25) (layer F.Cu) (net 3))
 (segment (start 134.62 113.284) (end 130.175 113.284) (width 0.25) (layer F.Cu) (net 3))
 (segment (start 140.335 111.515) (end 140.335 113.284) (width 0.25) (layer F.Cu) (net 3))
 (segment (start 141.859 113.284) (end 140.335 113.284) (width 0.25) (layer F.Cu) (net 3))
 (segment (start 137.795 112.19) (end 137.795 113.284) (width 0.25) (layer F.Cu) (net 3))
 (segment (start 137.795 111.515) (end 137.795 112.19) (width 0.25) (layer F.Cu) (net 3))
 (segment (start 140.335 113.284) (end 137.795 113.284) (width 0.25) (layer F.Cu) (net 3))
 (segment (start 137.795 113.284) (end 134.62 113.284) (width 0.25) (layer F.Cu) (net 3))
 (segment (start 142.494 113.284) (end 141.859 113.284) (width 0.25) (layer F.Cu) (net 3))
 (segment (start 142.56 111.59) (end 142.56 113.218) (width 0.25) (layer F.Cu) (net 3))
 (segment (start 142.56 113.218) (end 142.494 113.284) (width 0.25) (layer F.Cu) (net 3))
 (segment (start 151.13 112.141) (end 151.13 107.315) (width 0.25) (layer F.Cu) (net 3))
 (segment (start 143.51 113.284) (end 149.987 113.284) (width 0.25) (layer F.Cu) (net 3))
 (segment (start 149.987 113.284) (end 151.13 112.141) (width 0.25) (layer F.Cu) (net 3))
 (segment (start 129.225 99.67) (end 129.885 100.33) (width 0.25) (layer F.Cu) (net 7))
 (segment (start 129.225 98.89) (end 129.225 99.67) (width 0.25) (layer F.Cu) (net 7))
 (segment (start 146.685 100.33) (end 148.59 102.235) (width 0.25) (layer F.Cu) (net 7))
 (segment (start 148.59 102.235) (end 149.225 102.235) (width 0.25) (layer F.Cu) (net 7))
 (segment (start 131.445 99.99) (end 131.445 100.33) (width 0.25) (layer F.Cu) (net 7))
 (segment (start 131.125 99.67) (end 131.445 99.99) (width 0.25) (layer F.Cu) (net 7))
 (segment (start 131.125 98.89) (end 131.125 99.67) (width 0.25) (layer F.Cu) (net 7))
 (segment (start 129.885 100.33) (end 131.445 100.33) (width 0.25) (layer F.Cu) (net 7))
 (segment (start 131.445 100.33) (end 146.685 100.33) (width 0.25) (layer F.Cu) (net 7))
 (segment (start 143.755 105.8) (end 143.755 106.68) (width 0.25) (layer F.Cu) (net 4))
 (segment (start 144.78 104.775) (end 143.755 105.8) (width 0.25) (layer F.Cu) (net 4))
 (segment (start 145.415 104.775) (end 144.78 104.775) (width 0.25) (layer F.Cu) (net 4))
 (segment (start 149.225 103.505) (end 146.685 103.505) (width 0.25) (layer F.Cu) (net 4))
 (segment (start 146.685 103.505) (end 145.415 104.775) (width 0.25) (layer F.Cu) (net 4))
 (segment (start 144.78 103.87) (end 144.78 104.775) (width 0.25) (layer F.Cu) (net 4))
 (segment (start 141.85 106.68) (end 141.605 106.435) (width 0.25) (layer F.Cu) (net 4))
 (segment (start 143.755 106.68) (end 141.85 106.68) (width 0.25) (layer F.Cu) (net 4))
 (segment (start 141.535 106.365) (end 141.605 106.435) (width 0.25) (layer F.Cu) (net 4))
 (segment (start 139.43 106.365) (end 141.535 106.365) (width 0.25) (layer F.Cu) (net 4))
 (segment (start 109.465 111.125) (end 107.95 109.61) (width 0.25) (layer F.Cu) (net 12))
 (segment (start 107.95 109.61) (end 107.95 104.775) (width 0.25) (layer F.Cu) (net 12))
 (segment (start 107.95 104.775) (end 109.465 104.775) (width 0.25) (layer F.Cu) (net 12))
 (segment (start 85.09 101.6) (end 85.09 104.775) (width 0.25) (layer F.Cu) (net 12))
 (segment (start 85.09 104.775) (end 85.09 106.68) (width 0.25) (layer F.Cu) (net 12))
 (segment (start 107.95 104.775) (end 85.09 104.775) (width 0.25) (layer F.Cu) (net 12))
 (segment (start 111.515 104.775) (end 113.91 104.775) (width 0.25) (layer F.Cu) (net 10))
 (segment (start 148.59 106.045) (end 149.225 106.045) (width 0.25) (layer F.Cu) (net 6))
 (segment (start 144.46 109.39) (end 145.245 109.39) (width 0.25) (layer F.Cu) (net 6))
 (segment (start 145.245 109.39) (end 148.59 106.045) (width 0.25) (layer F.Cu) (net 6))
 (segment (start 144.46 110.81) (end 144.46 111.59) (width 0.25) (layer F.Cu) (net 2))
 (segment (start 133.35 110.49) (end 144.14 110.49) (width 0.25) (layer F.Cu) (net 2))
 (segment (start 144.14 110.49) (end 144.46 110.81) (width 0.25) (layer F.Cu) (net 2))
 (segment (start 130.175 107.705) (end 130.175 108.585) (width 0.25) (layer F.Cu) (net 2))
 (segment (start 130.175 109.465) (end 130.175 108.585) (width 0.25) (layer F.Cu) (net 2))
 (segment (start 130.175 108.585) (end 131.445 108.585) (width 0.25) (layer F.Cu) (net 2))
 (segment (start 131.445 108.585) (end 132.715 109.855) (width 0.25) (layer F.Cu) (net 2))
 (segment (start 133.67 110.81) (end 133.67 111.65) (width 0.25) (layer F.Cu) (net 2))
 (segment (start 133.35 110.49) (end 133.67 110.81) (width 0.25) (layer F.Cu) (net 2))
 (segment (start 132.715 109.855) (end 133.35 110.49) (width 0.25) (layer F.Cu) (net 2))
 (segment (start 140.015 95.565) (end 140.015 96.63) (width 0.25) (layer F.Cu) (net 9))
 (segment (start 139.065 94.615) (end 140.015 95.565) (width 0.25) (layer F.Cu) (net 9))
 (segment (start 129.225 96.69) (end 129.225 95.91) (width 0.25) (layer F.Cu) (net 9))
 (segment (start 129.225 95.91) (end 130.52 94.615) (width 0.25) (layer F.Cu) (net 9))
 (segment (start 143.23 96.63) (end 143.755 97.155) (width 0.25) (layer F.Cu) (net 9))
 (segment (start 140.015 96.63) (end 143.23 96.63) (width 0.25) (layer F.Cu) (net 9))
 (segment (start 132.42 94.615) (end 132.715 94.615) (width 0.25) (layer F.Cu) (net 9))
 (segment (start 131.125 95.91) (end 132.42 94.615) (width 0.25) (layer F.Cu) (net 9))
 (segment (start 131.125 96.69) (end 131.125 95.91) (width 0.25) (layer F.Cu) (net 9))
 (segment (start 130.52 94.615) (end 132.715 94.615) (width 0.25) (layer F.Cu) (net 9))
 (segment (start 132.715 94.615) (end 139.065 94.615) (width 0.25) (layer F.Cu) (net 9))
 (segment (start 145.805 97.155) (end 149.225 97.155) (width 0.25) (layer F.Cu) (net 15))
 (segment (start 115.96 111.125) (end 118.355 111.125) (width 0.25) (layer F.Cu) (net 14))
 (segment (start 111.515 111.125) (end 113.91 111.125) (width 0.25) (layer F.Cu) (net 13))
 (segment (start 115.96 104.775) (end 118.355 104.775) (width 0.25) (layer F.Cu) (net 11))
 (segment (start 132.96 102.235) (end 130.175 102.235) (width 0.25) (layer F.Cu) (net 1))
 (segment (start 137.48 107.315) (end 137.795 107.63) (width 0.25) (layer F.Cu) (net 1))
 (segment (start 137.43 107.315) (end 137.48 107.315) (width 0.25) (layer F.Cu) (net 1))
 (segment (start 137.795 107.63) (end 137.795 109.465) (width 0.25) (layer F.Cu) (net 1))
 (segment (start 134.62 107.315) (end 137.43 107.315) (width 0.25) (layer F.Cu) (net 1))
 (segment (start 134.62 109.33) (end 134.62 107.315) (width 0.25) (layer F.Cu) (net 1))
 (segment (start 130.175 105.655) (end 132.325 105.655) (width 0.25) (layer F.Cu) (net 1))
 (segment (start 132.325 105.655) (end 133.985 107.315) (width 0.25) (layer F.Cu) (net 1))
 (segment (start 133.985 107.315) (end 134.62 107.315) (width 0.25) (layer F.Cu) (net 1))
 (segment (start 137.795 109.465) (end 140.335 109.465) (width 0.25) (layer F.Cu) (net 1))
 (segment (start 143.51 108.61) (end 143.51 109.39) (width 0.25) (layer F.Cu) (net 1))
 (segment (start 143.434999 108.534999) (end 143.51 108.61) (width 0.25) (layer F.Cu) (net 1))
 (segment (start 141.265001 108.534999) (end 143.434999 108.534999) (width 0.25) (layer F.Cu) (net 1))
 (segment (start 140.335 109.465) (end 141.265001 108.534999) (width 0.25) (layer F.Cu) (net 1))
 (segment (start 126.365 105.655) (end 126.365 104.775) (width 0.25) (layer F.Cu) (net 1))
 (segment (start 127 104.14) (end 130.175 104.14) (width 0.25) (layer F.Cu) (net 1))
 (segment (start 126.365 104.775) (end 127 104.14) (width 0.25) (layer F.Cu) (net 1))
 (segment (start 130.175 102.235) (end 130.175 104.14) (width 0.25) (layer F.Cu) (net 1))
 (segment (start 130.175 104.14) (end 130.175 105.655) (width 0.25) (layer F.Cu) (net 1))
 (segment (start 122.555 104.775) (end 121.285 104.775) (width 0.25) (layer F.Cu) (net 2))
 (segment (start 121.285 104.775) (end 120.405 104.775) (width 0.25) (layer F.Cu) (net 2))
 (segment (start 126.365 108.585) (end 130.175 108.585) (width 0.25) (layer F.Cu) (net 2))
 (segment (start 126.365 108.585) (end 126.365 109.465) (width 0.25) (layer F.Cu) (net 2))
 (segment (start 126.365 107.705) (end 126.365 108.585) (width 0.25) (layer F.Cu) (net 2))
 (segment (start 126.365 108.585) (end 125.095 108.585) (width 0.25) (layer F.Cu) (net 2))
 (segment (start 125.095 108.585) (end 122.555 106.045) (width 0.25) (layer F.Cu) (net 2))
 (segment (start 122.555 106.045) (end 122.555 104.775) (width 0.25) (layer F.Cu) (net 2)))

